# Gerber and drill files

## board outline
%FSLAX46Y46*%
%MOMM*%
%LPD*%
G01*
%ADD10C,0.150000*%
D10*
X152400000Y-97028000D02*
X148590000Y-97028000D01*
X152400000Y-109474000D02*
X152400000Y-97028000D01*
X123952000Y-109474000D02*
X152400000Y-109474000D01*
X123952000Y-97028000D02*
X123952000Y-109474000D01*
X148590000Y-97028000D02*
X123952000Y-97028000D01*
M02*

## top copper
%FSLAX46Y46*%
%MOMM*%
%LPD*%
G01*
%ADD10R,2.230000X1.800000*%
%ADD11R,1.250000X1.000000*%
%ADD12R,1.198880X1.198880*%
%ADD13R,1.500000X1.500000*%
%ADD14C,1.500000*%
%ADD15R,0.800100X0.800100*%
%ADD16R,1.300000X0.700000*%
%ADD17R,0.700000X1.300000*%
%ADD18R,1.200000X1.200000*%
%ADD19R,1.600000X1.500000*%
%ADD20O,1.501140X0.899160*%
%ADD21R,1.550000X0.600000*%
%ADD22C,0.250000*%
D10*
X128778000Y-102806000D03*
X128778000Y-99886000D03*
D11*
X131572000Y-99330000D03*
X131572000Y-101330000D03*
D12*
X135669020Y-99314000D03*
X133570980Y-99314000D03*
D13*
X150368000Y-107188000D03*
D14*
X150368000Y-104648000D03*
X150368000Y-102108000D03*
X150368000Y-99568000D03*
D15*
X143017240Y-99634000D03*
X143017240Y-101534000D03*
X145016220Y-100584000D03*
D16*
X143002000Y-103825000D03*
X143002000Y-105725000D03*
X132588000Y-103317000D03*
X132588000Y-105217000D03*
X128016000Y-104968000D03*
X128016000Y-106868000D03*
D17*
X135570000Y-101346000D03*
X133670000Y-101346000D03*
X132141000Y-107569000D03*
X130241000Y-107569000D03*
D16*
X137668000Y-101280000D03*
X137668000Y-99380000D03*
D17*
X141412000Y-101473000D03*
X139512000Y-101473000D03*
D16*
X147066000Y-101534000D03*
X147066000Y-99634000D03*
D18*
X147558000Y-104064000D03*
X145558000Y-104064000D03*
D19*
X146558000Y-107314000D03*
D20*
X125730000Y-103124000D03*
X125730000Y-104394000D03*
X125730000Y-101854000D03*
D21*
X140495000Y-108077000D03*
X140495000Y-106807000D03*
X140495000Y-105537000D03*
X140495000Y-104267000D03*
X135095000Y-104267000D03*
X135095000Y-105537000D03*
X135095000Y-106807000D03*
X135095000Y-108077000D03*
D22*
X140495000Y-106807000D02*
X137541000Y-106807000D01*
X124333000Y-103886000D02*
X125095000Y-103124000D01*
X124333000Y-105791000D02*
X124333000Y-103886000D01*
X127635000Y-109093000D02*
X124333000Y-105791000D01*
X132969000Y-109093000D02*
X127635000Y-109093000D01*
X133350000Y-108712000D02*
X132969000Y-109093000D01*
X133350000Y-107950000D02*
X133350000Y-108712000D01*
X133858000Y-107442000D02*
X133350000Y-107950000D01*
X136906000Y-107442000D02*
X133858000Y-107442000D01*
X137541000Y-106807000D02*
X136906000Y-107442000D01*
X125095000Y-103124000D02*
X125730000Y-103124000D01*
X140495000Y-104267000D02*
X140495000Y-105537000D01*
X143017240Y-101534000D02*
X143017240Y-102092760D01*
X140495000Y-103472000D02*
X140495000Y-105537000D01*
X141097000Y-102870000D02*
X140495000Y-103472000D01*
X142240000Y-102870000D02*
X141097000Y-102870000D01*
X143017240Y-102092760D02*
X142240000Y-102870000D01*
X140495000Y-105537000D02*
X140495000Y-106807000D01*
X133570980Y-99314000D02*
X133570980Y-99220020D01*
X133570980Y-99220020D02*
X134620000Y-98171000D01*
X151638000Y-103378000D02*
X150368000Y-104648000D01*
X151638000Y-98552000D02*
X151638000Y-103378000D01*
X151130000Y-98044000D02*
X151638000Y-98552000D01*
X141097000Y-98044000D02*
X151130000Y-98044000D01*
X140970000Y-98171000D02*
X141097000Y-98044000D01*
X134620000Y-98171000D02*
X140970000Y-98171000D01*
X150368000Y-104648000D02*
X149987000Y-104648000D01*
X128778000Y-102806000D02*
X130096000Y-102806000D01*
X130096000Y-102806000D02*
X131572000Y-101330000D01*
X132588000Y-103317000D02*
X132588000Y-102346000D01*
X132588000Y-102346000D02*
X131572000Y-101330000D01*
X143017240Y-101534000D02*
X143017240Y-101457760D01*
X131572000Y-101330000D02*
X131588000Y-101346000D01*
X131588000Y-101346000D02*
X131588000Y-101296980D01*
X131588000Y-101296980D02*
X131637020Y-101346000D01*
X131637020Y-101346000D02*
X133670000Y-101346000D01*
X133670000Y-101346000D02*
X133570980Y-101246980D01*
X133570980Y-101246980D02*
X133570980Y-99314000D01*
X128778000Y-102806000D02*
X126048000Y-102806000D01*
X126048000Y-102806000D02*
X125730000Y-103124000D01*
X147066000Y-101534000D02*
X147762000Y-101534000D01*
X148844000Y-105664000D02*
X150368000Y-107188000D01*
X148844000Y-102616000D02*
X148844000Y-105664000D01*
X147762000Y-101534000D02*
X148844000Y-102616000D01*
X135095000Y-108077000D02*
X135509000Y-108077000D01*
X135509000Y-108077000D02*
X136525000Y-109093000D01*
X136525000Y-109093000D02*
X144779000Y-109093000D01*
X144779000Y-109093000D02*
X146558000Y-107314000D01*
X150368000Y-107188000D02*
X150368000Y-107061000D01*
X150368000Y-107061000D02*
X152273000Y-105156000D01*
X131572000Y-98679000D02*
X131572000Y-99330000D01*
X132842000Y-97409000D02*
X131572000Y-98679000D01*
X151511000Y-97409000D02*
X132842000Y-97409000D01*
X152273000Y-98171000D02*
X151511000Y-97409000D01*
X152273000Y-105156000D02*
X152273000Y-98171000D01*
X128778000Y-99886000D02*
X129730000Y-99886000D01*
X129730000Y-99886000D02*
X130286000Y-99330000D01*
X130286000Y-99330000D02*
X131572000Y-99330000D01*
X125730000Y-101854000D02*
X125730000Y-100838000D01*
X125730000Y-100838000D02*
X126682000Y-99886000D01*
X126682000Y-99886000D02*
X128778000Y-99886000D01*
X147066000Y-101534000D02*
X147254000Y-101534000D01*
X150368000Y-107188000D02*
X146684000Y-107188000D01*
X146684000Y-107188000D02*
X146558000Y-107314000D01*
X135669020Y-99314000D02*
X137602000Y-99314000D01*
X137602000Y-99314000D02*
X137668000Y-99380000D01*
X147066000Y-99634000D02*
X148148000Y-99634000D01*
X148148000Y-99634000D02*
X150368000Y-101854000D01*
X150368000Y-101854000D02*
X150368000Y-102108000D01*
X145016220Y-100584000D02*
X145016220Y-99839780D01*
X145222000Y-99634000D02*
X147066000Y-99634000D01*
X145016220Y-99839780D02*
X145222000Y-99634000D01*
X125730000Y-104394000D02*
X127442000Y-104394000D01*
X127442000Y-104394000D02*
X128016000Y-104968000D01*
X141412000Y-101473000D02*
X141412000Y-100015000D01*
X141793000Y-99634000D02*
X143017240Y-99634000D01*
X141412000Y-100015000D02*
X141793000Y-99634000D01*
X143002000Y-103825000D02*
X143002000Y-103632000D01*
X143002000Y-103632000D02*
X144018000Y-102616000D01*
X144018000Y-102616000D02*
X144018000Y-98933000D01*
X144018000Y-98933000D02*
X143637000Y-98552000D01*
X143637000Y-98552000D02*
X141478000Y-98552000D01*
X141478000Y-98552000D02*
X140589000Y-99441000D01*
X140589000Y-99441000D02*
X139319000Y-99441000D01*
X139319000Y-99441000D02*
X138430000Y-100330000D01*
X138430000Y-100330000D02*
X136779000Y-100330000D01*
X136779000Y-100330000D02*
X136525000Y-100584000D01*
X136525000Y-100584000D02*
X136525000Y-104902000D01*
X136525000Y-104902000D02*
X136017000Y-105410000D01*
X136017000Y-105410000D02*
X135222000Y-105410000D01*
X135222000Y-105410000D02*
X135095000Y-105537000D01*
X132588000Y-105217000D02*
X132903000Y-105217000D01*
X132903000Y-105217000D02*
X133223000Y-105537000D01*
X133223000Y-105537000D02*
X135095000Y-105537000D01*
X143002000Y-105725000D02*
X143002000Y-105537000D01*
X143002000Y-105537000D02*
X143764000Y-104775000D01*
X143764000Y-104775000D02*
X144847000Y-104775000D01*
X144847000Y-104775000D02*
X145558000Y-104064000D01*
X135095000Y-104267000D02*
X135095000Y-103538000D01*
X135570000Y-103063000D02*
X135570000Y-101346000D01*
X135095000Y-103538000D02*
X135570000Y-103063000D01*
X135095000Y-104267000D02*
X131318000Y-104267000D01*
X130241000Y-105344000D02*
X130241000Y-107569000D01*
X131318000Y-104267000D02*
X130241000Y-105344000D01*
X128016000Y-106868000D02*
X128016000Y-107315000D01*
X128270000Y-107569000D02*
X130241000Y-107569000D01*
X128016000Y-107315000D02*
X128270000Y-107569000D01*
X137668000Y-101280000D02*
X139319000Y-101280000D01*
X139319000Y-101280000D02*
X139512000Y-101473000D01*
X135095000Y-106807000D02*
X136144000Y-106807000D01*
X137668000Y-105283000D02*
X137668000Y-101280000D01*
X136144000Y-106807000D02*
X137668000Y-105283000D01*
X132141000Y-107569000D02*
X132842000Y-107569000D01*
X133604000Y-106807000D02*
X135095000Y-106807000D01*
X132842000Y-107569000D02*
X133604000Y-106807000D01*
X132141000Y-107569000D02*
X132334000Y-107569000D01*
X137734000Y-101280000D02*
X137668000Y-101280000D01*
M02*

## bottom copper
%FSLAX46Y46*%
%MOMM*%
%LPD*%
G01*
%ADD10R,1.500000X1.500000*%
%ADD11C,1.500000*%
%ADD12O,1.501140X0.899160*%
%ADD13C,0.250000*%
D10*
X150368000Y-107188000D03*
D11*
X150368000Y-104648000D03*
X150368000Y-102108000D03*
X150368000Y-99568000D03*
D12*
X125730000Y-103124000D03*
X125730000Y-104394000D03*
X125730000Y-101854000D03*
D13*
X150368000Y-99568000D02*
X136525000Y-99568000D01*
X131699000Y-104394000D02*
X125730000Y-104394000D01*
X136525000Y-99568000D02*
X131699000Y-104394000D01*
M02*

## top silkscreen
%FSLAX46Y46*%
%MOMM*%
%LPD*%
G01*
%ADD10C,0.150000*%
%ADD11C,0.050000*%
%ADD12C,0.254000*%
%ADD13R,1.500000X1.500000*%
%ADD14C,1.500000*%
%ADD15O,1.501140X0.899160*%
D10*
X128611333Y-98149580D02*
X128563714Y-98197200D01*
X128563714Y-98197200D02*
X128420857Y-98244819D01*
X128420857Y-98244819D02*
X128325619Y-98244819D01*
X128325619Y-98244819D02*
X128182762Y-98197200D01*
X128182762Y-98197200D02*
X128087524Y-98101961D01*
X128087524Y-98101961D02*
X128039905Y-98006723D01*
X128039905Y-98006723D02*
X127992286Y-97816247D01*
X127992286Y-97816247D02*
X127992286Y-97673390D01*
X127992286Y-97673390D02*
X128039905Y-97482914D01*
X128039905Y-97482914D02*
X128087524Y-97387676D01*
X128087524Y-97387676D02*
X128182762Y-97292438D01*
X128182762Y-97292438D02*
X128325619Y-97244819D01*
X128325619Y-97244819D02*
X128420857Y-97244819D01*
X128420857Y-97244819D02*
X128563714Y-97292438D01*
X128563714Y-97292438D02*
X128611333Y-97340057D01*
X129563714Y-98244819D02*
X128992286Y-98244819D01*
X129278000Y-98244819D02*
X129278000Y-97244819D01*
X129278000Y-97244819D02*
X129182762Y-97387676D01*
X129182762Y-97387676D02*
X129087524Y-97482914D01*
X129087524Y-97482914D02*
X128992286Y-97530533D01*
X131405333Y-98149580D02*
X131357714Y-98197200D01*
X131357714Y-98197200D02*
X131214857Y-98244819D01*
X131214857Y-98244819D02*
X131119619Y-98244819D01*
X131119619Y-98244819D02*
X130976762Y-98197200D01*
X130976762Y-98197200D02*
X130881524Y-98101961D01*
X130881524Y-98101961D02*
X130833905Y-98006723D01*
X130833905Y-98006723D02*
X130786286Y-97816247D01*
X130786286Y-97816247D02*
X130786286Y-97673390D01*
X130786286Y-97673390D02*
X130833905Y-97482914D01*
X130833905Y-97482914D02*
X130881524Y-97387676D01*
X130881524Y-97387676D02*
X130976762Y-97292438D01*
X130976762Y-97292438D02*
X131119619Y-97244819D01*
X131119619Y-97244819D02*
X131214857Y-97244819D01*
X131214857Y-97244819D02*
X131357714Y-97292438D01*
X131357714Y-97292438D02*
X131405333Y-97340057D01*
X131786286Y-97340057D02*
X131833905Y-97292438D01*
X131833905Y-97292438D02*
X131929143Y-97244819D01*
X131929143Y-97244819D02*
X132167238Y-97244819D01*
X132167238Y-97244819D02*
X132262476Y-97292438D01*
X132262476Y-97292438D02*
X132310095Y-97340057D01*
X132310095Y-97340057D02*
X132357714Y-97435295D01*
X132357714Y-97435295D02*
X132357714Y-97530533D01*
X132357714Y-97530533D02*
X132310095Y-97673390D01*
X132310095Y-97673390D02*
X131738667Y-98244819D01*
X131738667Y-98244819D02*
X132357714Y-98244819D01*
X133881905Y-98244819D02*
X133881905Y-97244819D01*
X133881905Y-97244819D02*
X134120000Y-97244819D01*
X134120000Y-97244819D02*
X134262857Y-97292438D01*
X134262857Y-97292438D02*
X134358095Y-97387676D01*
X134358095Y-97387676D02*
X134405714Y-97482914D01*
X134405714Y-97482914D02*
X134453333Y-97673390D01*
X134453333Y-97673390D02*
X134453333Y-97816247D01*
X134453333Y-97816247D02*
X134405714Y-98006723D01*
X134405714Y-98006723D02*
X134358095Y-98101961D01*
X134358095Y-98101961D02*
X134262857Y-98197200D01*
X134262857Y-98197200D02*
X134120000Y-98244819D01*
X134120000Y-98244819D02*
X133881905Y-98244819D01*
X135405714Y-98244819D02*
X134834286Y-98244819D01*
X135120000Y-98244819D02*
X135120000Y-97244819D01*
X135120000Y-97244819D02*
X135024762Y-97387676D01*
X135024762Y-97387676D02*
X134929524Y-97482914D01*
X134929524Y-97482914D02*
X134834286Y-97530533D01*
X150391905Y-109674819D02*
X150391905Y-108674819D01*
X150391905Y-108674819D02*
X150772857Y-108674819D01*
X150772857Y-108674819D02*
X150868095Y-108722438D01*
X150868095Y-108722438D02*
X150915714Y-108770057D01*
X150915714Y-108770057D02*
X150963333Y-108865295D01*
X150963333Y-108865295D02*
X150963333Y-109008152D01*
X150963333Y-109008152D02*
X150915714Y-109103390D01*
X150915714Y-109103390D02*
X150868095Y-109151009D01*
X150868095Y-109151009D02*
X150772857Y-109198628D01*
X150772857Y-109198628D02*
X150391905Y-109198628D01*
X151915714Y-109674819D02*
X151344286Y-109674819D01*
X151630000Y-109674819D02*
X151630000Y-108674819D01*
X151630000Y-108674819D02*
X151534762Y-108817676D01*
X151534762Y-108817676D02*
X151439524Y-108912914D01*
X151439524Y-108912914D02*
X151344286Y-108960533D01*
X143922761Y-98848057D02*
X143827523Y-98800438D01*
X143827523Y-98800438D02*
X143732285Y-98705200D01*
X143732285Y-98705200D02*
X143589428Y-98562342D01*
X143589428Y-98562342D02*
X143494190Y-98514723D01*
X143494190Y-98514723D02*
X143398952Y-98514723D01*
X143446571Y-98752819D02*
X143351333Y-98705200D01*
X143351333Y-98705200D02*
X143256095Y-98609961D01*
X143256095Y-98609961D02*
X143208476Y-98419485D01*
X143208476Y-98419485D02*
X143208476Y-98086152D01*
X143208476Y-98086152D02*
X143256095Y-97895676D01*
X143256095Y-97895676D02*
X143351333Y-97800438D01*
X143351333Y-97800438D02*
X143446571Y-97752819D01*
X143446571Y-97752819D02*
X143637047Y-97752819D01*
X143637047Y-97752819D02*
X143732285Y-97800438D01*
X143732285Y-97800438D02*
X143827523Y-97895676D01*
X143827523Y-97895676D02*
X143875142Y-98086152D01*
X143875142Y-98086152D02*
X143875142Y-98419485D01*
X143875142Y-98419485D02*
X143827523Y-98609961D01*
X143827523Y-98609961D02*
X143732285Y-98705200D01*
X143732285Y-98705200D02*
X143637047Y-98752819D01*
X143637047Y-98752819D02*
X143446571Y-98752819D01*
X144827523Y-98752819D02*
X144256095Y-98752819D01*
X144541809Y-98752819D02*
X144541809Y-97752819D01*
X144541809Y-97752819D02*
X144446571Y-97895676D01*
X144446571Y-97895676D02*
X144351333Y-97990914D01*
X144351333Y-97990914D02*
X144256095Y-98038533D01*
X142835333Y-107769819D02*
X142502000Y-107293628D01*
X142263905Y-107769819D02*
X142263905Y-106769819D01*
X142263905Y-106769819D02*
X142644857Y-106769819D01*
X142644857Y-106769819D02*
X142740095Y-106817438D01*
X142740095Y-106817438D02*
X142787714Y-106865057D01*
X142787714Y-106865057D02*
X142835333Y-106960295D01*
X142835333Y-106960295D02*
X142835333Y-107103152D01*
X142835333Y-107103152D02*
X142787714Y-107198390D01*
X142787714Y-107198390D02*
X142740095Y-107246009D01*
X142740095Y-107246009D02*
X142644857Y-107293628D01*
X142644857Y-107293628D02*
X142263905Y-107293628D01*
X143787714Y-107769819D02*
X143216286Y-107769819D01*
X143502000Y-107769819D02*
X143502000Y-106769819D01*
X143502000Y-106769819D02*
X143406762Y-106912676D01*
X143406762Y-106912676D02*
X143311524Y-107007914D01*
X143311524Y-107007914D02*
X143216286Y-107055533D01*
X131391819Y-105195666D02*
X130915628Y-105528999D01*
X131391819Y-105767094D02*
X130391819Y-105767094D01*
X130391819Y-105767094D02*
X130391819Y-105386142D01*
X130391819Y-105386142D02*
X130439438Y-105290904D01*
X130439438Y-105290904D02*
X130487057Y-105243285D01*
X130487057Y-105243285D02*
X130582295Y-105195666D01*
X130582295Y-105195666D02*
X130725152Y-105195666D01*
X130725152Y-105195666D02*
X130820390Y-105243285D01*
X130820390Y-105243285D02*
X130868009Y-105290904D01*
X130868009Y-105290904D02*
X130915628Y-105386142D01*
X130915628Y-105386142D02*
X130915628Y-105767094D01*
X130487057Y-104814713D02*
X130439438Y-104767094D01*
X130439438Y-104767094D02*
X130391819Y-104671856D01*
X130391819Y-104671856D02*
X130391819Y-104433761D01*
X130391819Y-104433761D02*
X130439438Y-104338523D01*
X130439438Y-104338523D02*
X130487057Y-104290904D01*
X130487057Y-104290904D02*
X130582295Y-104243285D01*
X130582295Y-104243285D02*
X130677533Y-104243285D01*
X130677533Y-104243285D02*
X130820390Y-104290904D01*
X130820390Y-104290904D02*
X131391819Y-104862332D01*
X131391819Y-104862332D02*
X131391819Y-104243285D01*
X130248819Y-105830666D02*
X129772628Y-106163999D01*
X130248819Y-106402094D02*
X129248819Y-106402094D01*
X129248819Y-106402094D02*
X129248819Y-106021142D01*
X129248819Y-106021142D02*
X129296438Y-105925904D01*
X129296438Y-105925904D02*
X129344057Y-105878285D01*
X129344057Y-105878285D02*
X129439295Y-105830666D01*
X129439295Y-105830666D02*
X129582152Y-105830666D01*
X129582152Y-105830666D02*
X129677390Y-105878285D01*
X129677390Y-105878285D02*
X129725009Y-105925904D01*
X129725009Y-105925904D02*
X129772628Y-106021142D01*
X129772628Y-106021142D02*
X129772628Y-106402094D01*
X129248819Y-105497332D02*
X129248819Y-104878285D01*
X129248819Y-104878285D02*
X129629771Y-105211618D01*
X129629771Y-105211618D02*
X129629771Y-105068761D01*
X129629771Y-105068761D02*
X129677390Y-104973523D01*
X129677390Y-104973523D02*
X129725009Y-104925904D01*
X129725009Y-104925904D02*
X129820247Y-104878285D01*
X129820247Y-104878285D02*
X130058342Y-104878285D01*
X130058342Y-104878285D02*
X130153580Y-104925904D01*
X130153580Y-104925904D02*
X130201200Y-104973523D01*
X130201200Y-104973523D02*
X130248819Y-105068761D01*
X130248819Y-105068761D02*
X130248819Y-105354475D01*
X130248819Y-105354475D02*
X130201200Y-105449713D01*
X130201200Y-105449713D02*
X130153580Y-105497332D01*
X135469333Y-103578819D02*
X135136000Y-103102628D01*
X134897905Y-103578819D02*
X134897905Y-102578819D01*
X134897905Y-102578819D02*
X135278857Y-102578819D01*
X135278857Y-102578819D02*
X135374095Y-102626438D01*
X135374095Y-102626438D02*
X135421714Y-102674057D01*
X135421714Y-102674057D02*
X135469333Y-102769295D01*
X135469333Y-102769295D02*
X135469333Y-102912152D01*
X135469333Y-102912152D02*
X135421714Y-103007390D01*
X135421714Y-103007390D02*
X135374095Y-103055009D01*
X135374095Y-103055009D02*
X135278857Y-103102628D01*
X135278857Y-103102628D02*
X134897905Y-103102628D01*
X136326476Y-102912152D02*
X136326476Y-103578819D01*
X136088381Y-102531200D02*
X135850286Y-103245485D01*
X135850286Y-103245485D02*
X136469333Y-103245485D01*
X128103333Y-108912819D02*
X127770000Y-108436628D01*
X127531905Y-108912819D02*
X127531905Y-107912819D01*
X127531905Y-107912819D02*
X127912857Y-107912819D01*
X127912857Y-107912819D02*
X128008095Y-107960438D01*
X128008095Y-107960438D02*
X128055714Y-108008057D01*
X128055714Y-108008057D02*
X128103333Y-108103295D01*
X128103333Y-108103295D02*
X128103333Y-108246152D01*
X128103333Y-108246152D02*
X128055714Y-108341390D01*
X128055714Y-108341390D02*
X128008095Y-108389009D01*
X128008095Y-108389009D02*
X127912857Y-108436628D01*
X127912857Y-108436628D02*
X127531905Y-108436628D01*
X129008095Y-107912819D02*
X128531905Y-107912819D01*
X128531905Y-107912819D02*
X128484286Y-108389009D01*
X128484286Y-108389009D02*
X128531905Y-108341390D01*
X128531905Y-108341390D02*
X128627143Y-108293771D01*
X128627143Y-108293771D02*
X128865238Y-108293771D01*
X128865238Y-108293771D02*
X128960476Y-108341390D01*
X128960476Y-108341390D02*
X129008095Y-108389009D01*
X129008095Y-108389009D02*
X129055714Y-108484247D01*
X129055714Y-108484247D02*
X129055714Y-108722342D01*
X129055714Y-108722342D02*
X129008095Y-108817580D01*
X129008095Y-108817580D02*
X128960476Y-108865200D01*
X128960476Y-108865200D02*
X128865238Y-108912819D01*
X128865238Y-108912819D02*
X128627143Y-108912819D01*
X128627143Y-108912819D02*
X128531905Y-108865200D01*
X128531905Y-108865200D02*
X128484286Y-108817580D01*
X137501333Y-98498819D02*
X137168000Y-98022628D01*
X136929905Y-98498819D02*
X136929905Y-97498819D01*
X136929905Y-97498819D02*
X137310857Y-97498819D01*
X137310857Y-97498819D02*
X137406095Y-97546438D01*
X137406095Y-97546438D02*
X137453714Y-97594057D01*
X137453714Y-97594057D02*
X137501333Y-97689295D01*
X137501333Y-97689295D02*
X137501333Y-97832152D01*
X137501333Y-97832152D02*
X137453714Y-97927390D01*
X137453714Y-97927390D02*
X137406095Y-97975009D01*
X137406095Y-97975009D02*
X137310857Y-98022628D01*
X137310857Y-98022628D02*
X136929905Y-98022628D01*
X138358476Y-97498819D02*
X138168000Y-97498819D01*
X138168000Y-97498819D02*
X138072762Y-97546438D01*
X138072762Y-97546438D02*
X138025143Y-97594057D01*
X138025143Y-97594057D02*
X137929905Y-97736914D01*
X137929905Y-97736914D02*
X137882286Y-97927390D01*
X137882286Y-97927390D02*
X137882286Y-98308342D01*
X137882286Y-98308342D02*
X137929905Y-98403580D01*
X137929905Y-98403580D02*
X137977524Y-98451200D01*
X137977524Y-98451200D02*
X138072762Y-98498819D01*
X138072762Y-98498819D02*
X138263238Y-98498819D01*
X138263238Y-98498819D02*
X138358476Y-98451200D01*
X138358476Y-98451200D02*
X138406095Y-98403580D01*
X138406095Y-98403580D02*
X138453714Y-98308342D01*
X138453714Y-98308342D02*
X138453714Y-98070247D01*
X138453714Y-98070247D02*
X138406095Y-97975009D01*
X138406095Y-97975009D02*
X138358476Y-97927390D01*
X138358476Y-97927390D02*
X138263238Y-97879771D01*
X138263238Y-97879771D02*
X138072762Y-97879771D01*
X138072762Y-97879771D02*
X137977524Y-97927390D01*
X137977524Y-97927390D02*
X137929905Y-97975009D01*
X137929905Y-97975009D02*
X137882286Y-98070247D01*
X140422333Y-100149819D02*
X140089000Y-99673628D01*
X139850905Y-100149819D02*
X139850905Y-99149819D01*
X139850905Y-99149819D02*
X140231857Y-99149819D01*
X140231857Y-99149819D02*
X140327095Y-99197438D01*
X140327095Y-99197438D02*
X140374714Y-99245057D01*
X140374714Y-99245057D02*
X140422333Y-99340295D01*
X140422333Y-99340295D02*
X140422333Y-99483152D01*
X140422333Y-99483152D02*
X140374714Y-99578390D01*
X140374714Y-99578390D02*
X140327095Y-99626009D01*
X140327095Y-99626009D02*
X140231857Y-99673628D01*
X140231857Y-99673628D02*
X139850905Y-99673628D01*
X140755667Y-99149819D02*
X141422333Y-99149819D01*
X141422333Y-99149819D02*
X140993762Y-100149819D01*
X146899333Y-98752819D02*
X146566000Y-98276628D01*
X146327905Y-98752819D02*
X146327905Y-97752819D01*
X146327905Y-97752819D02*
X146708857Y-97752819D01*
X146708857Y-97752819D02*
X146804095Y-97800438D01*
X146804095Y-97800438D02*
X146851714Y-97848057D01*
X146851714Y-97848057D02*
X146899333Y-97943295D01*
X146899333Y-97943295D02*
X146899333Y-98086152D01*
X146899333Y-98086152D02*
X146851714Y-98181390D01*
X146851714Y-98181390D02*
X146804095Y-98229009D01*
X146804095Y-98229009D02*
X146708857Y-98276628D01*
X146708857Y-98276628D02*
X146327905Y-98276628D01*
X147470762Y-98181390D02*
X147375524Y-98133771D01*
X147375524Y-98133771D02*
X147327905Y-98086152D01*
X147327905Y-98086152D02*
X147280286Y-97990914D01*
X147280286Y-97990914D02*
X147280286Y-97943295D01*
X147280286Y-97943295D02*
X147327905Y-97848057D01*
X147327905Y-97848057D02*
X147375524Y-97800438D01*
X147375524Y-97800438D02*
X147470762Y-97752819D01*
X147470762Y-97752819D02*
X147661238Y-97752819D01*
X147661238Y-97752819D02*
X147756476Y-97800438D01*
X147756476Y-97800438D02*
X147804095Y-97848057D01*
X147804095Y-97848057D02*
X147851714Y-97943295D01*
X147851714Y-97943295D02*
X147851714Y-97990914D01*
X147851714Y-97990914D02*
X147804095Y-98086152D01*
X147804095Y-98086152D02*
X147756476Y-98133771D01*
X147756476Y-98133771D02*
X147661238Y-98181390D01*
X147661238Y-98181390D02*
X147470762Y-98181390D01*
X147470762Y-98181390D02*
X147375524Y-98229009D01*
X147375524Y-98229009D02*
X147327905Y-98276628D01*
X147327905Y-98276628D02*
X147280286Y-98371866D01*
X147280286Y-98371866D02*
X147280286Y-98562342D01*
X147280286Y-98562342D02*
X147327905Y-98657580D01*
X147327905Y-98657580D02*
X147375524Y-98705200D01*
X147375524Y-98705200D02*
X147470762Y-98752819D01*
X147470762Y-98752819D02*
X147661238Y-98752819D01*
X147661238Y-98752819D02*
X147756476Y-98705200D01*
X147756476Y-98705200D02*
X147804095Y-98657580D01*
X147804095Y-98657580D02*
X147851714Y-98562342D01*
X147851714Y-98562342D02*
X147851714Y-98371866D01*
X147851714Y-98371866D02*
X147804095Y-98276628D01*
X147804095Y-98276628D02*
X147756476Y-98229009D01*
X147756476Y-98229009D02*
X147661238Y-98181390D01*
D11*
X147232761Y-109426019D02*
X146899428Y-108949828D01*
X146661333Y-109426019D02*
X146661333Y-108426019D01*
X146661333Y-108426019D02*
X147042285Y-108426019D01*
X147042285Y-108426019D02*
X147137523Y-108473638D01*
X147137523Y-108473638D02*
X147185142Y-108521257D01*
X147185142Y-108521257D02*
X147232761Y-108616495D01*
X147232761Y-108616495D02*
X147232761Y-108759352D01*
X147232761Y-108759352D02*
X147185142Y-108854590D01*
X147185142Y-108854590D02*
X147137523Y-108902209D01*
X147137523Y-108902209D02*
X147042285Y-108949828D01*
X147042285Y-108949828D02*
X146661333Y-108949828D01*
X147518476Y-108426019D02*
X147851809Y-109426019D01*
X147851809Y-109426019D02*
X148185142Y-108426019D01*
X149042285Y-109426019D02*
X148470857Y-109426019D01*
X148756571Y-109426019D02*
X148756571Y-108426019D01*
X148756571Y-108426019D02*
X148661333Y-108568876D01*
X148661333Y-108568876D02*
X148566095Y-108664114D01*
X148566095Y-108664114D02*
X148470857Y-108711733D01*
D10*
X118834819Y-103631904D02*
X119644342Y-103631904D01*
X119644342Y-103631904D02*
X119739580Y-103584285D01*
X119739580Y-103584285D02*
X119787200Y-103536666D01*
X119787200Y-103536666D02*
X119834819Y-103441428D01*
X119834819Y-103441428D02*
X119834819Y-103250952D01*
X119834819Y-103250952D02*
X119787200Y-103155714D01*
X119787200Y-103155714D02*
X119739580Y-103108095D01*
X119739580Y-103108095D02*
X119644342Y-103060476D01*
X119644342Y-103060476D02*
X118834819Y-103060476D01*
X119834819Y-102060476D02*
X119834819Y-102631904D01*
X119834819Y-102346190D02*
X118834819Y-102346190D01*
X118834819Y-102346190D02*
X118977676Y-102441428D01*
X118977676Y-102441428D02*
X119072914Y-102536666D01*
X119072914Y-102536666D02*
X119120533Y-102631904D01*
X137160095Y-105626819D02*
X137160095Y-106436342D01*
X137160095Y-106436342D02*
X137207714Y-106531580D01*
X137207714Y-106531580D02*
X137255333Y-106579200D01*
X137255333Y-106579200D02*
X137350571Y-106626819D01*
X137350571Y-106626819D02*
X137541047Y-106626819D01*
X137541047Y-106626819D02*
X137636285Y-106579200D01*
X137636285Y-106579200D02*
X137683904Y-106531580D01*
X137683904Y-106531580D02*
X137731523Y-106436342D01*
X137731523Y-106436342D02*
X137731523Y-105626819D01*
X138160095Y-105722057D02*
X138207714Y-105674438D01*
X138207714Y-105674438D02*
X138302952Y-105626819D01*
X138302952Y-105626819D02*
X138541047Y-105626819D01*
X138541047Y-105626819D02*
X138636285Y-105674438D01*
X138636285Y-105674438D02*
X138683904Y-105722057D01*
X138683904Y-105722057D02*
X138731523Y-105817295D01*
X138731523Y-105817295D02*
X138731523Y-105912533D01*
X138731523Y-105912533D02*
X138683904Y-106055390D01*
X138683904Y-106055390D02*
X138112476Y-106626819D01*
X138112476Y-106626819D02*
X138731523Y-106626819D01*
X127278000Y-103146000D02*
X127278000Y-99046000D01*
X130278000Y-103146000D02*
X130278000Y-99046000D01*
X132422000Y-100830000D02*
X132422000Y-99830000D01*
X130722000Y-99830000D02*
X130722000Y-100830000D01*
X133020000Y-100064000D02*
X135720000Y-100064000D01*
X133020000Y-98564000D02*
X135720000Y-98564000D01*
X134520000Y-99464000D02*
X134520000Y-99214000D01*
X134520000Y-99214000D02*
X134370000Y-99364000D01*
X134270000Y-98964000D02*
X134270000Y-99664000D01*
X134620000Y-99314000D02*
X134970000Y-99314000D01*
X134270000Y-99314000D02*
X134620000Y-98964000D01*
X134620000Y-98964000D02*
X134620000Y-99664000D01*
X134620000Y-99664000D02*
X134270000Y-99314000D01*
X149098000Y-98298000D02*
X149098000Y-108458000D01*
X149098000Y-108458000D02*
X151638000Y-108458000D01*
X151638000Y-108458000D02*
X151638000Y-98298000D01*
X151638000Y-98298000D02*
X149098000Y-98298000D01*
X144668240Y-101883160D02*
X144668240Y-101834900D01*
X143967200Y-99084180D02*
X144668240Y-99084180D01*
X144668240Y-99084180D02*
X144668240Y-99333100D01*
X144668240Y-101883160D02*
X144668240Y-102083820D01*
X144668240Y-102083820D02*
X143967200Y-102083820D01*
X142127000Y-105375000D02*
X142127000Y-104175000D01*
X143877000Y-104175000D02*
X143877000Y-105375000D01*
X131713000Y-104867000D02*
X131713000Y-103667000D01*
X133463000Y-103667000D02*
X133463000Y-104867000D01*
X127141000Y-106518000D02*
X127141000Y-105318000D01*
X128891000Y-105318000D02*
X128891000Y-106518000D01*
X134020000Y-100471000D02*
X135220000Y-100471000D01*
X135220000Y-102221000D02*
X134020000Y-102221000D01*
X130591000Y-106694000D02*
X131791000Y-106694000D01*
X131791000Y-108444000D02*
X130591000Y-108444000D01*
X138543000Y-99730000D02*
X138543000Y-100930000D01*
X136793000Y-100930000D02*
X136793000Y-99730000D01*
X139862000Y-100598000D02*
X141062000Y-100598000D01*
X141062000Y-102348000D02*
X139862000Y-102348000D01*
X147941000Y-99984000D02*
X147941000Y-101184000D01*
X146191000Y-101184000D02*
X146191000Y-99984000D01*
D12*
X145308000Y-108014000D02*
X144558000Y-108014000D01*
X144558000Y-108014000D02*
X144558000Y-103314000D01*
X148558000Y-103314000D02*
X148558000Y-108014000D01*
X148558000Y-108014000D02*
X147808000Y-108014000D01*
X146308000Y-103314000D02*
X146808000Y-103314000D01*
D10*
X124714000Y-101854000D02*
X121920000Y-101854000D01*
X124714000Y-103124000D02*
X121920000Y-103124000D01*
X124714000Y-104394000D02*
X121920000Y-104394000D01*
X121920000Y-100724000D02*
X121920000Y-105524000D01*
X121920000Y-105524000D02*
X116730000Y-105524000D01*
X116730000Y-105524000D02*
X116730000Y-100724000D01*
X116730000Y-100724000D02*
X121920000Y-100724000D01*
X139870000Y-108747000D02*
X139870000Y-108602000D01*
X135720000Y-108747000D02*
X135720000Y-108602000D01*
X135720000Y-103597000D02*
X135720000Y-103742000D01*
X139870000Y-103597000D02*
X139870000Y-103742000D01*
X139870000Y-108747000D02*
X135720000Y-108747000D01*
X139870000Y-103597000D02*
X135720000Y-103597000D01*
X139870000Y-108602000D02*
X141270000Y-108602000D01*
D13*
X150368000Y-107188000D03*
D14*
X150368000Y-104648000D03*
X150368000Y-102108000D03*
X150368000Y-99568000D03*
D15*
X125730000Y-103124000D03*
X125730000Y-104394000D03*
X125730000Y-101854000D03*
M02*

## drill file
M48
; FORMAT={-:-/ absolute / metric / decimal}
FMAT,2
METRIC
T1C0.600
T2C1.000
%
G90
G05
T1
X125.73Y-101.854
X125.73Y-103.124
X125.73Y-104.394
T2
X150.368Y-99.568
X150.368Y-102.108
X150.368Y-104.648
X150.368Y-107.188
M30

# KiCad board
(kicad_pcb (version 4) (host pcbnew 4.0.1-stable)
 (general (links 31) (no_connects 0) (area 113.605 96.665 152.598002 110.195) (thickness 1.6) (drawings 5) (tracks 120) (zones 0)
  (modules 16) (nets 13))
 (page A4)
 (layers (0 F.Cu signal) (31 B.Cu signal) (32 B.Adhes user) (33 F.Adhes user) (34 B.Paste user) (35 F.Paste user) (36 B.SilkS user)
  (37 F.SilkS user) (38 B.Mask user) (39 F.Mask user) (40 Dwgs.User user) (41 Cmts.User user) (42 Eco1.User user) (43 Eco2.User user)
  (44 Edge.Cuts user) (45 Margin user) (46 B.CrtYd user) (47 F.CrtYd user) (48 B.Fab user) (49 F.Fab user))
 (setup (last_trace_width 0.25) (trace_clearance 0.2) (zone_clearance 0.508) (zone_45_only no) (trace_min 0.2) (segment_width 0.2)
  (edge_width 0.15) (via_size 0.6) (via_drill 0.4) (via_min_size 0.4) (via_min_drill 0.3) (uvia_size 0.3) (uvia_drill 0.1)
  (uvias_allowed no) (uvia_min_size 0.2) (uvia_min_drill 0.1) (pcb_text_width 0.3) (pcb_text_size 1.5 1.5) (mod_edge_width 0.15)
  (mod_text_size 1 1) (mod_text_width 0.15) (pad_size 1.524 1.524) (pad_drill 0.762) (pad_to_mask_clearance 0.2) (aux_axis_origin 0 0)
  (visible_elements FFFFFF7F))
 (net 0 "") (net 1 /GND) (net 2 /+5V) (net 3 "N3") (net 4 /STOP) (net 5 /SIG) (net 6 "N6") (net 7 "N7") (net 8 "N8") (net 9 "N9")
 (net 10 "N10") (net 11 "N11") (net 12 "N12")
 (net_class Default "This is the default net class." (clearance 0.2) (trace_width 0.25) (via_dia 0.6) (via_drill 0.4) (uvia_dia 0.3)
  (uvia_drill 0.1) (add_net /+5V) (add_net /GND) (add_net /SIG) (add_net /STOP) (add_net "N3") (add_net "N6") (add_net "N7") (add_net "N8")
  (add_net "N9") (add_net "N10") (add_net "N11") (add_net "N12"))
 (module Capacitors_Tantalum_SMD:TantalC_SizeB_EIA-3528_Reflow (layer F.Cu) (at 128.778 101.346 270)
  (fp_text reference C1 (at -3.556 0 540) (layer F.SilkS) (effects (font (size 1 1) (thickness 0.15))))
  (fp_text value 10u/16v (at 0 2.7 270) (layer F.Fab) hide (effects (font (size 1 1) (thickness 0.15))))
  (fp_line (start 1.8 1.5) (end -2.3 1.5) (layer F.SilkS) (width 0.15))
  (fp_line (start 1.8 -1.5) (end -2.3 -1.5) (layer F.SilkS) (width 0.15))
  (pad 2 smd rect (at 1.46 0 270) (size 1.8 2.23) (layers F.Cu F.Paste F.Mask) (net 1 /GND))
  (pad 1 smd rect (at -1.46 0 270) (size 1.8 2.23) (layers F.Cu F.Paste F.Mask) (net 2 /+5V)))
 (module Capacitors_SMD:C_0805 (layer F.Cu) (at 131.572 100.33 270)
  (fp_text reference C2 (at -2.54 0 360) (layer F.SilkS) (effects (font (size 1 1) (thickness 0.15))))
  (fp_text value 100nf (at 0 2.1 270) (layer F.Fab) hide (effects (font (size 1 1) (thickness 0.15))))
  (fp_line (start 0.5 -0.85) (end -0.5 -0.85) (layer F.SilkS) (width 0.15))
  (fp_line (start -0.5 0.85) (end 0.5 0.85) (layer F.SilkS) (width 0.15))
  (pad 1 smd rect (at -1 0 270) (size 1 1.25) (layers F.Cu F.Paste F.Mask) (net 2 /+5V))
  (pad 2 smd rect (at 1 0 270) (size 1 1.25) (layers F.Cu F.Paste F.Mask) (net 1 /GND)))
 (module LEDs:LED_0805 (layer F.Cu) (at 134.62 99.314)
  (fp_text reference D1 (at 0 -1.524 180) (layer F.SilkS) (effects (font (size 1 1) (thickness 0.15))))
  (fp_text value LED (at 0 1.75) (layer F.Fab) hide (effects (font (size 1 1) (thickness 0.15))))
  (fp_line (start -1.6 0.75) (end 1.1 0.75) (layer F.SilkS) (width 0.15))
  (fp_line (start -1.6 -0.75) (end 1.1 -0.75) (layer F.SilkS) (width 0.15))
  (fp_line (start -0.1 0.15) (end -0.1 -0.1) (layer F.SilkS) (width 0.15))
  (fp_line (start -0.1 -0.1) (end -0.25 0.05) (layer F.SilkS) (width 0.15))
  (fp_line (start -0.35 -0.35) (end -0.35 0.35) (layer F.SilkS) (width 0.15))
  (fp_line (start 0 0) (end 0.35 0) (layer F.SilkS) (width 0.15))
  (fp_line (start -0.35 0) (end 0 -0.35) (layer F.SilkS) (width 0.15))
  (fp_line (start 0 -0.35) (end 0 0.35) (layer F.SilkS) (width 0.15))
  (fp_line (start 0 0.35) (end -0.35 0) (layer F.SilkS) (width 0.15))
  (pad 2 smd rect (at 1.04902 0 180) (size 1.19888 1.19888) (layers F.Cu F.Paste F.Mask) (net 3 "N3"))
  (pad 1 smd rect (at -1.04902 0 180) (size 1.19888 1.19888) (layers F.Cu F.Paste F.Mask) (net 1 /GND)))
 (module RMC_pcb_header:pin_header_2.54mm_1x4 (layer F.Cu) (at 150.368 103.378 90)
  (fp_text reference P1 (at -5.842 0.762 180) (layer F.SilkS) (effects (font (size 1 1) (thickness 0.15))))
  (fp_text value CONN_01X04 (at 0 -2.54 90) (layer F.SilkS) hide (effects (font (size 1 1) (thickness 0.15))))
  (fp_line (start 5.08 -1.27) (end -5.08 -1.27) (layer F.SilkS) (width 0.15))
  (fp_line (start -5.08 -1.27) (end -5.08 1.27) (layer F.SilkS) (width 0.15))
  (fp_line (start -5.08 1.27) (end 5.08 1.27) (layer F.SilkS) (width 0.15))
  (fp_line (start 5.08 1.27) (end 5.08 -1.27) (layer F.SilkS) (width 0.15))
  (pad 1 thru_hole rect (at -3.81 0 90) (size 1.5 1.5) (drill 1) (layers *.Cu *.Mask F.SilkS) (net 2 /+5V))
  (pad 2 thru_hole circle (at -1.27 0 90) (size 1.5 1.5) (drill 1) (layers *.Cu *.Mask F.SilkS) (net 1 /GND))
  (pad 3 thru_hole circle (at 1.27 0 90) (size 1.5 1.5) (drill 1) (layers *.Cu *.Mask F.SilkS) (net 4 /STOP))
  (pad 4 thru_hole circle (at 3.81 0 90) (size 1.5 1.5) (drill 1) (layers *.Cu *.Mask F.SilkS) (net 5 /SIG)))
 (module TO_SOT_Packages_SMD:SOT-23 (layer F.Cu) (at 144.018 100.584 270)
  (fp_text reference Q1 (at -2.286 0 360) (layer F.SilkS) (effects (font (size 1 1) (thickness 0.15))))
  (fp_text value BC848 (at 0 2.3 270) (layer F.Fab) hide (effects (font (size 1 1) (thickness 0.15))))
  (fp_line (start 1.29916 -0.65024) (end 1.2509 -0.65024) (layer F.SilkS) (width 0.15))
  (fp_line (start -1.49982 0.0508) (end -1.49982 -0.65024) (layer F.SilkS) (width 0.15))
  (fp_line (start -1.49982 -0.65024) (end -1.2509 -0.65024) (layer F.SilkS) (width 0.15))
  (fp_line (start 1.29916 -0.65024) (end 1.49982 -0.65024) (layer F.SilkS) (width 0.15))
  (fp_line (start 1.49982 -0.65024) (end 1.49982 0.0508) (layer F.SilkS) (width 0.15))
  (pad 1 smd rect (at -0.95 1.00076 270) (size 0.8001 0.8001) (layers F.Cu F.Paste F.Mask) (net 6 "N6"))
  (pad 2 smd rect (at 0.95 1.00076 270) (size 0.8001 0.8001) (layers F.Cu F.Paste F.Mask) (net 1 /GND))
  (pad 3 smd rect (at 0 -0.99822 270) (size 0.8001 0.8001) (layers F.Cu F.Paste F.Mask) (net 4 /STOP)))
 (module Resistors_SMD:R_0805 (layer F.Cu) (at 143.002 104.775 270)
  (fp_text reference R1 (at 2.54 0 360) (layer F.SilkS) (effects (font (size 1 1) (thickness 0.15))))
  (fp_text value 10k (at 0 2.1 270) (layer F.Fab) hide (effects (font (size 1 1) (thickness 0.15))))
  (fp_line (start 0.6 0.875) (end -0.6 0.875) (layer F.SilkS) (width 0.15))
  (fp_line (start -0.6 -0.875) (end 0.6 -0.875) (layer F.SilkS) (width 0.15))
  (pad 1 smd rect (at -0.95 0 270) (size 0.7 1.3) (layers F.Cu F.Paste F.Mask) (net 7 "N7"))
  (pad 2 smd rect (at 0.95 0 270) (size 0.7 1.3) (layers F.Cu F.Paste F.Mask) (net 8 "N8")))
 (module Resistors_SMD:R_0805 (layer F.Cu) (at 132.588 104.267 270)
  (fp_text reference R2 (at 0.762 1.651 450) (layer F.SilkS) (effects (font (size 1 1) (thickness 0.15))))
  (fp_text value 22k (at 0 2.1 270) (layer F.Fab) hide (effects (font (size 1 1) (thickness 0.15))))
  (fp_line (start 0.6 0.875) (end -0.6 0.875) (layer F.SilkS) (width 0.15))
  (fp_line (start -0.6 -0.875) (end 0.6 -0.875) (layer F.SilkS) (width 0.15))
  (pad 1 smd rect (at -0.95 0 270) (size 0.7 1.3) (layers F.Cu F.Paste F.Mask) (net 1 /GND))
  (pad 2 smd rect (at 0.95 0 270) (size 0.7 1.3) (layers F.Cu F.Paste F.Mask) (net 7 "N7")))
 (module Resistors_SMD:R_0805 (layer F.Cu) (at 128.016 105.918 270)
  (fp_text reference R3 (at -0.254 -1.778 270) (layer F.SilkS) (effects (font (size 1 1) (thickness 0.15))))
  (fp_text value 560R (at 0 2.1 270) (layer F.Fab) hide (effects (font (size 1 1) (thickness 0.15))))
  (fp_line (start 0.6 0.875) (end -0.6 0.875) (layer F.SilkS) (width 0.15))
  (fp_line (start -0.6 -0.875) (end 0.6 -0.875) (layer F.SilkS) (width 0.15))
  (pad 1 smd rect (at -0.95 0 270) (size 0.7 1.3) (layers F.Cu F.Paste F.Mask) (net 5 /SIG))
  (pad 2 smd rect (at 0.95 0 270) (size 0.7 1.3) (layers F.Cu F.Paste F.Mask) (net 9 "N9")))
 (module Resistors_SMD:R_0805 (layer F.Cu) (at 134.62 101.346 180)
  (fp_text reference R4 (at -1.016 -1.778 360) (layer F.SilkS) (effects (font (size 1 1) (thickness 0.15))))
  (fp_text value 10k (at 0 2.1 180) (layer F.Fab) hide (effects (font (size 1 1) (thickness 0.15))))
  (fp_line (start 0.6 0.875) (end -0.6 0.875) (layer F.SilkS) (width 0.15))
  (fp_line (start -0.6 -0.875) (end 0.6 -0.875) (layer F.SilkS) (width 0.15))
  (pad 1 smd rect (at -0.95 0 180) (size 0.7 1.3) (layers F.Cu F.Paste F.Mask) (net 9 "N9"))
  (pad 2 smd rect (at 0.95 0 180) (size 0.7 1.3) (layers F.Cu F.Paste F.Mask) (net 1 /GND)))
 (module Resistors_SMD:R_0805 (layer F.Cu) (at 131.191 107.569 180)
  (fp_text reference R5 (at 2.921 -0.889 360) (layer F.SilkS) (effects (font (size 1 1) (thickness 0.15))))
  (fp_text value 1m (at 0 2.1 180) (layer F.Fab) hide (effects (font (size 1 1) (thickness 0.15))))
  (fp_line (start 0.6 0.875) (end -0.6 0.875) (layer F.SilkS) (width 0.15))
  (fp_line (start -0.6 -0.875) (end 0.6 -0.875) (layer F.SilkS) (width 0.15))
  (pad 1 smd rect (at -0.95 0 180) (size 0.7 1.3) (layers F.Cu F.Paste F.Mask) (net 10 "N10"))
  (pad 2 smd rect (at 0.95 0 180) (size 0.7 1.3) (layers F.Cu F.Paste F.Mask) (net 9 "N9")))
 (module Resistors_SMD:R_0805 (layer F.Cu) (at 137.668 100.33 90)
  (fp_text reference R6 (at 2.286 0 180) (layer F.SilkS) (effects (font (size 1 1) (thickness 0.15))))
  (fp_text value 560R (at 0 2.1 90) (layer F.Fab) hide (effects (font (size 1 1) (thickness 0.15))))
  (fp_line (start 0.6 0.875) (end -0.6 0.875) (layer F.SilkS) (width 0.15))
  (fp_line (start -0.6 -0.875) (end 0.6 -0.875) (layer F.SilkS) (width 0.15))
  (pad 1 smd rect (at -0.95 0 90) (size 0.7 1.3) (layers F.Cu F.Paste F.Mask) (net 10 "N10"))
  (pad 2 smd rect (at 0.95 0 90) (size 0.7 1.3) (layers F.Cu F.Paste F.Mask) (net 3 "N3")))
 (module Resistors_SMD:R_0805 (layer F.Cu) (at 140.462 101.473 180)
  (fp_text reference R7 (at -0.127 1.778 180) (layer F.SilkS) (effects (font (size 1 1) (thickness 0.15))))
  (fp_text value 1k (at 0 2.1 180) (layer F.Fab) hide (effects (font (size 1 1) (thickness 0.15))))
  (fp_line (start 0.6 0.875) (end -0.6 0.875) (layer F.SilkS) (width 0.15))
  (fp_line (start -0.6 -0.875) (end 0.6 -0.875) (layer F.SilkS) (width 0.15))
  (pad 1 smd rect (at -0.95 0 180) (size 0.7 1.3) (layers F.Cu F.Paste F.Mask) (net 6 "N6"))
  (pad 2 smd rect (at 0.95 0 180) (size 0.7 1.3) (layers F.Cu F.Paste F.Mask) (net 10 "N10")))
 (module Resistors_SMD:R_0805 (layer F.Cu) (at 147.066 100.584 90)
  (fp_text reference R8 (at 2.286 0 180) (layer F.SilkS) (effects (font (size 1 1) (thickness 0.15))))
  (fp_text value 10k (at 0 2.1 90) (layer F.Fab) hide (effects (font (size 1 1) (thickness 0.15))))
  (fp_line (start 0.6 0.875) (end -0.6 0.875) (layer F.SilkS) (width 0.15))
  (fp_line (start -0.6 -0.875) (end 0.6 -0.875) (layer F.SilkS) (width 0.15))
  (pad 1 smd rect (at -0.95 0 90) (size 0.7 1.3) (layers F.Cu F.Paste F.Mask) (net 2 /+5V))
  (pad 2 smd rect (at 0.95 0 90) (size 0.7 1.3) (layers F.Cu F.Paste F.Mask) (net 4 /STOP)))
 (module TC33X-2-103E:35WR (layer F.Cu) (at 146.558 105.664 180) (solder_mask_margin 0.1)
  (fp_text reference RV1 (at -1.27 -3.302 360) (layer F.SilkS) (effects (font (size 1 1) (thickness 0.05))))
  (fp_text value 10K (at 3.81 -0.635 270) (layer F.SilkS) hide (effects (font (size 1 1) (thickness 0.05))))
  (fp_line (start 1.25 -2.35) (end 2 -2.35) (layer F.SilkS) (width 0.254))
  (fp_line (start 2 -2.35) (end 2 2.35) (layer F.SilkS) (width 0.254))
  (fp_line (start -2 2.35) (end -2 -2.35) (layer F.SilkS) (width 0.254))
  (fp_line (start -2 -2.35) (end -1.25 -2.35) (layer F.SilkS) (width 0.254))
  (fp_line (start 0.25 2.35) (end -0.25 2.35) (layer F.SilkS) (width 0.254))
  (pad 1 smd rect (at -1 1.6 180) (size 1.2 1.2) (layers F.Cu F.Paste F.Mask) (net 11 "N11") (solder_mask_margin 0.2))
  (pad 3 smd rect (at 1 1.6 180) (size 1.2 1.2) (layers F.Cu F.Paste F.Mask) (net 8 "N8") (solder_mask_margin 0.2))
  (pad 2 smd rect (at 0 -1.65 180) (size 1.6 1.5) (layers F.Cu F.Paste F.Mask) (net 2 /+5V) (solder_mask_margin 0.2)))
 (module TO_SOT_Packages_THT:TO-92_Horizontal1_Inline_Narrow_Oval (layer F.Cu) (at 125.73 101.854 270)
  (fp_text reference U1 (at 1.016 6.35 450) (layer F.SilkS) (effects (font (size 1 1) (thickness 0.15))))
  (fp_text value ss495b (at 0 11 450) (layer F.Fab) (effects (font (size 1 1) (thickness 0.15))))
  (fp_line (start 0 1.016) (end 0 3.81) (layer F.SilkS) (width 0.15))
  (fp_line (start 1.27 1.016) (end 1.27 3.81) (layer F.SilkS) (width 0.15))
  (fp_line (start 2.54 1.016) (end 2.54 3.81) (layer F.SilkS) (width 0.15))
  (fp_line (start -1.13 3.81) (end 3.67 3.81) (layer F.SilkS) (width 0.15))
  (fp_line (start 3.67 3.81) (end 3.67 9) (layer F.SilkS) (width 0.15))
  (fp_line (start 3.67 9) (end -1.13 9) (layer F.SilkS) (width 0.15))
  (fp_line (start -1.13 9) (end -1.13 3.81) (layer F.SilkS) (width 0.15))
  (pad 2 thru_hole oval (at 1.27 0 90) (size 0.89916 1.50114) (drill 0.6) (layers *.Cu *.Mask F.SilkS) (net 1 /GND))
  (pad 3 thru_hole oval (at 2.54 0 90) (size 0.89916 1.50114) (drill 0.6) (layers *.Cu *.Mask F.SilkS) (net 5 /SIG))
  (pad 1 thru_hole oval (at 0 0 90) (size 0.89916 1.50114) (drill 0.6) (layers *.Cu *.Mask F.SilkS) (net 2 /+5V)))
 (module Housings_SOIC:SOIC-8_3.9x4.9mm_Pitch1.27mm (layer F.Cu) (at 137.795 106.172 180)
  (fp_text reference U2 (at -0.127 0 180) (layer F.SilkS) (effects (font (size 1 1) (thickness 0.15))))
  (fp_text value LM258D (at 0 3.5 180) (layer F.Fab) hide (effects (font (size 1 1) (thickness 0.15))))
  (fp_line (start -2.075 -2.575) (end -2.075 -2.43) (layer F.SilkS) (width 0.15))
  (fp_line (start 2.075 -2.575) (end 2.075 -2.43) (layer F.SilkS) (width 0.15))
  (fp_line (start 2.075 2.575) (end 2.075 2.43) (layer F.SilkS) (width 0.15))
  (fp_line (start -2.075 2.575) (end -2.075 2.43) (layer F.SilkS) (width 0.15))
  (fp_line (start -2.075 -2.575) (end 2.075 -2.575) (layer F.SilkS) (width 0.15))
  (fp_line (start -2.075 2.575) (end 2.075 2.575) (layer F.SilkS) (width 0.15))
  (fp_line (start -2.075 -2.43) (end -3.475 -2.43) (layer F.SilkS) (width 0.15))
  (pad 1 smd rect (at -2.7 -1.905 180) (size 1.55 0.6) (layers F.Cu F.Paste F.Mask) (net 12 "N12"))
  (pad 2 smd rect (at -2.7 -0.635 180) (size 1.55 0.6) (layers F.Cu F.Paste F.Mask) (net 1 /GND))
  (pad 3 smd rect (at -2.7 0.635 180) (size 1.55 0.6) (layers F.Cu F.Paste F.Mask) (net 1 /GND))
  (pad 4 smd rect (at -2.7 1.905 180) (size 1.55 0.6) (layers F.Cu F.Paste F.Mask) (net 1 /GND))
  (pad 5 smd rect (at 2.7 1.905 180) (size 1.55 0.6) (layers F.Cu F.Paste F.Mask) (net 9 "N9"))
  (pad 6 smd rect (at 2.7 0.635 180) (size 1.55 0.6) (layers F.Cu F.Paste F.Mask) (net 7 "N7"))
  (pad 7 smd rect (at 2.7 -0.635 180) (size 1.55 0.6) (layers F.Cu F.Paste F.Mask) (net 10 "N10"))
  (pad 8 smd rect (at 2.7 -1.905 180) (size 1.55 0.6) (layers F.Cu F.Paste F.Mask) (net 2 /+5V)))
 (gr_line (start 152.4 97.028) (end 148.59 97.028) (angle 90) (layer Edge.Cuts) (width 0.15))
 (gr_line (start 152.4 109.474) (end 152.4 97.028) (angle 90) (layer Edge.Cuts) (width 0.15))
 (gr_line (start 123.952 109.474) (end 152.4 109.474) (angle 90) (layer Edge.Cuts) (width 0.15))
 (gr_line (start 123.952 97.028) (end 123.952 109.474) (angle 90) (layer Edge.Cuts) (width 0.15))
 (gr_line (start 148.59 97.028) (end 123.952 97.028) (angle 90) (layer Edge.Cuts) (width 0.15))
 (segment (start 140.495 106.807) (end 137.541 106.807) (width 0.25) (layer F.Cu) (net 1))
 (segment (start 124.333 103.886) (end 125.095 103.124) (width 0.25) (layer F.Cu) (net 1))
 (segment (start 124.333 105.791) (end 124.333 103.886) (width 0.25) (layer F.Cu) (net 1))
 (segment (start 127.635 109.093) (end 124.333 105.791) (width 0.25) (layer F.Cu) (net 1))
 (segment (start 132.969 109.093) (end 127.635 109.093) (width 0.25) (layer F.Cu) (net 1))
 (segment (start 133.35 108.712) (end 132.969 109.093) (width 0.25) (layer F.Cu) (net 1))
 (segment (start 133.35 107.95) (end 133.35 108.712) (width 0.25) (layer F.Cu) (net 1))
 (segment (start 133.858 107.442) (end 133.35 107.95) (width 0.25) (layer F.Cu) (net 1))
 (segment (start 136.906 107.442) (end 133.858 107.442) (width 0.25) (layer F.Cu) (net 1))
 (segment (start 137.541 106.807) (end 136.906 107.442) (width 0.25) (layer F.Cu) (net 1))
 (segment (start 125.095 103.124) (end 125.73 103.124) (width 0.25) (layer F.Cu) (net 1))
 (segment (start 140.495 104.267) (end 140.495 105.537) (width 0.25) (layer F.Cu) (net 1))
 (segment (start 143.01724 101.534) (end 143.01724 102.09276) (width 0.25) (layer F.Cu) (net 1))
 (segment (start 140.495 103.472) (end 140.495 105.537) (width 0.25) (layer F.Cu) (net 1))
 (segment (start 141.097 102.87) (end 140.495 103.472) (width 0.25) (layer F.Cu) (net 1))
 (segment (start 142.24 102.87) (end 141.097 102.87) (width 0.25) (layer F.Cu) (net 1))
 (segment (start 143.01724 102.09276) (end 142.24 102.87) (width 0.25) (layer F.Cu) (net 1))
 (segment (start 140.495 105.537) (end 140.495 106.807) (width 0.25) (layer F.Cu) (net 1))
 (segment (start 133.57098 99.314) (end 133.57098 99.22002) (width 0.25) (layer F.Cu) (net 1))
 (segment (start 133.57098 99.22002) (end 134.62 98.171) (width 0.25) (layer F.Cu) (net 1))
 (segment (start 151.638 103.378) (end 150.368 104.648) (width 0.25) (layer F.Cu) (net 1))
 (segment (start 151.638 98.552) (end 151.638 103.378) (width 0.25) (layer F.Cu) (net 1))
 (segment (start 151.13 98.044) (end 151.638 98.552) (width 0.25) (layer F.Cu) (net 1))
 (segment (start 141.097 98.044) (end 151.13 98.044) (width 0.25) (layer F.Cu) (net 1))
 (segment (start 140.97 98.171) (end 141.097 98.044) (width 0.25) (layer F.Cu) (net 1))
 (segment (start 134.62 98.171) (end 140.97 98.171) (width 0.25) (layer F.Cu) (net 1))
 (segment (start 150.368 104.648) (end 149.987 104.648) (width 0.25) (layer F.Cu) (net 1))
 (segment (start 128.778 102.806) (end 130.096 102.806) (width 0.25) (layer F.Cu) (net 1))
 (segment (start 130.096 102.806) (end 131.572 101.33) (width 0.25) (layer F.Cu) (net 1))
 (segment (start 132.588 103.317) (end 132.588 102.346) (width 0.25) (layer F.Cu) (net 1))
 (segment (start 132.588 102.346) (end 131.572 101.33) (width 0.25) (layer F.Cu) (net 1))
 (segment (start 143.01724 101.534) (end 143.01724 101.45776) (width 0.25) (layer F.Cu) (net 1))
 (segment (start 131.572 101.33) (end 131.588 101.346) (width 0.25) (layer F.Cu) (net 1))
 (segment (start 131.588 101.346) (end 131.588 101.29698) (width 0.25) (layer F.Cu) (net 1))
 (segment (start 131.588 101.29698) (end 131.63702 101.346) (width 0.25) (layer F.Cu) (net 1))
 (segment (start 131.63702 101.346) (end 133.67 101.346) (width 0.25) (layer F.Cu) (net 1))
 (segment (start 133.67 101.346) (end 133.57098 101.24698) (width 0.25) (layer F.Cu) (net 1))
 (segment (start 133.57098 101.24698) (end 133.57098 99.314) (width 0.25) (layer F.Cu) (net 1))
 (segment (start 128.778 102.806) (end 126.048 102.806) (width 0.25) (layer F.Cu) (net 1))
 (segment (start 126.048 102.806) (end 125.73 103.124) (width 0.25) (layer F.Cu) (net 1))
 (segment (start 147.066 101.534) (end 147.762 101.534) (width 0.25) (layer F.Cu) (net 2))
 (segment (start 148.844 105.664) (end 150.368 107.188) (width 0.25) (layer F.Cu) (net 2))
 (segment (start 148.844 102.616) (end 148.844 105.664) (width 0.25) (layer F.Cu) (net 2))
 (segment (start 147.762 101.534) (end 148.844 102.616) (width 0.25) (layer F.Cu) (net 2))
 (segment (start 135.095 108.077) (end 135.509 108.077) (width 0.25) (layer F.Cu) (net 2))
 (segment (start 135.509 108.077) (end 136.525 109.093) (width 0.25) (layer F.Cu) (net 2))
 (segment (start 136.525 109.093) (end 144.779 109.093) (width 0.25) (layer F.Cu) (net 2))
 (segment (start 144.779 109.093) (end 146.558 107.314) (width 0.25) (layer F.Cu) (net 2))
 (segment (start 150.368 107.188) (end 150.368 107.061) (width 0.25) (layer F.Cu) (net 2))
 (segment (start 150.368 107.061) (end 152.273 105.156) (width 0.25) (layer F.Cu) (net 2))
 (segment (start 131.572 98.679) (end 131.572 99.33) (width 0.25) (layer F.Cu) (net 2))
 (segment (start 132.842 97.409) (end 131.572 98.679) (width 0.25) (layer F.Cu) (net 2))
 (segment (start 151.511 97.409) (end 132.842 97.409) (width 0.25) (layer F.Cu) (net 2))
 (segment (start 152.273 98.171) (end 151.511 97.409) (width 0.25) (layer F.Cu) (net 2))
 (segment (start 152.273 105.156) (end 152.273 98.171) (width 0.25) (layer F.Cu) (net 2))
 (segment (start 128.778 99.886) (end 129.73 99.886) (width 0.25) (layer F.Cu) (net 2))
 (segment (start 129.73 99.886) (end 130.286 99.33) (width 0.25) (layer F.Cu) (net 2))
 (segment (start 130.286 99.33) (end 131.572 99.33) (width 0.25) (layer F.Cu) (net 2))
 (segment (start 125.73 101.854) (end 125.73 100.838) (width 0.25) (layer F.Cu) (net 2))
 (segment (start 125.73 100.838) (end 126.682 99.886) (width 0.25) (layer F.Cu) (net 2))
 (segment (start 126.682 99.886) (end 128.778 99.886) (width 0.25) (layer F.Cu) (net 2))
 (segment (start 147.066 101.534) (end 147.254 101.534) (width 0.25) (layer F.Cu) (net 2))
 (segment (start 150.368 107.188) (end 146.684 107.188) (width 0.25) (layer F.Cu) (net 2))
 (segment (start 146.684 107.188) (end 146.558 107.314) (width 0.25) (layer F.Cu) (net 2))
 (segment (start 135.66902 99.314) (end 137.602 99.314) (width 0.25) (layer F.Cu) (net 3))
 (segment (start 137.602 99.314) (end 137.668 99.38) (width 0.25) (layer F.Cu) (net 3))
 (segment (start 147.066 99.634) (end 148.148 99.634) (width 0.25) (layer F.Cu) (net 4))
 (segment (start 148.148 99.634) (end 150.368 101.854) (width 0.25) (layer F.Cu) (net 4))
 (segment (start 150.368 101.854) (end 150.368 102.108) (width 0.25) (layer F.Cu) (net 4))
 (segment (start 145.01622 100.584) (end 145.01622 99.83978) (width 0.25) (layer F.Cu) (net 4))
 (segment (start 145.222 99.634) (end 147.066 99.634) (width 0.25) (layer F.Cu) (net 4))
 (segment (start 145.01622 99.83978) (end 145.222 99.634) (width 0.25) (layer F.Cu) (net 4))
 (segment (start 150.368 99.568) (end 136.525 99.568) (width 0.25) (layer B.Cu) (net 5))
 (segment (start 131.699 104.394) (end 125.73 104.394) (width 0.25) (layer B.Cu) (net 5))
 (segment (start 136.525 99.568) (end 131.699 104.394) (width 0.25) (layer B.Cu) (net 5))
 (segment (start 125.73 104.394) (end 127.442 104.394) (width 0.25) (layer F.Cu) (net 5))
 (segment (start 127.442 104.394) (end 128.016 104.968) (width 0.25) (layer F.Cu) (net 5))
 (segment (start 141.412 101.473) (end 141.412 100.015) (width 0.25) (layer F.Cu) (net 6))
 (segment (start 141.793 99.634) (end 143.01724 99.634) (width 0.25) (layer F.Cu) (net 6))
 (segment (start 141.412 100.015) (end 141.793 99.634) (width 0.25) (layer F.Cu) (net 6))
 (segment (start 143.002 103.825) (end 143.002 103.632) (width 0.25) (layer F.Cu) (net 7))
 (segment (start 143.002 103.632) (end 144.018 102.616) (width 0.25) (layer F.Cu) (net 7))
 (segment (start 144.018 102.616) (end 144.018 98.933) (width 0.25) (layer F.Cu) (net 7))
 (segment (start 144.018 98.933) (end 143.637 98.552) (width 0.25) (layer F.Cu) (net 7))
 (segment (start 143.637 98.552) (end 141.478 98.552) (width 0.25) (layer F.Cu) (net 7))
 (segment (start 141.478 98.552) (end 140.589 99.441) (width 0.25) (layer F.Cu) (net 7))
 (segment (start 140.589 99.441) (end 139.319 99.441) (width 0.25) (layer F.Cu) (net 7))
 (segment (start 139.319 99.441) (end 138.43 100.33) (width 0.25) (layer F.Cu) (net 7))
 (segment (start 138.43 100.33) (end 136.779 100.33) (width 0.25) (layer F.Cu) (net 7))
 (segment (start 136.779 100.33) (end 136.525 100.584) (width 0.25) (layer F.Cu) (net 7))
 (segment (start 136.525 100.584) (end 136.525 104.902) (width 0.25) (layer F.Cu) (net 7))
 (segment (start 136.525 104.902) (end 136.017 105.41) (width 0.25) (layer F.Cu) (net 7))
 (segment (start 136.017 105.41) (end 135.222 105.41) (width 0.25) (layer F.Cu) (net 7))
 (segment (start 135.222 105.41) (end 135.095 105.537) (width 0.25) (layer F.Cu) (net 7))
 (segment (start 132.588 105.217) (end 132.903 105.217) (width 0.25) (layer F.Cu) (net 7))
 (segment (start 132.903 105.217) (end 133.223 105.537) (width 0.25) (layer F.Cu) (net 7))
 (segment (start 133.223 105.537) (end 135.095 105.537) (width 0.25) (layer F.Cu) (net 7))
 (segment (start 143.002 105.725) (end 143.002 105.537) (width 0.25) (layer F.Cu) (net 8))
 (segment (start 143.002 105.537) (end 143.764 104.775) (width 0.25) (layer F.Cu) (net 8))
 (segment (start 143.764 104.775) (end 144.847 104.775) (width 0.25) (layer F.Cu) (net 8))
 (segment (start 144.847 104.775) (end 145.558 104.064) (width 0.25) (layer F.Cu) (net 8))
 (segment (start 135.095 104.267) (end 135.095 103.538) (width 0.25) (layer F.Cu) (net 9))
 (segment (start 135.57 103.063) (end 135.57 101.346) (width 0.25) (layer F.Cu) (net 9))
 (segment (start 135.095 103.538) (end 135.57 103.063) (width 0.25) (layer F.Cu) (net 9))
 (segment (start 135.095 104.267) (end 131.318 104.267) (width 0.25) (layer F.Cu) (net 9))
 (segment (start 130.241 105.344) (end 130.241 107.569) (width 0.25) (layer F.Cu) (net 9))
 (segment (start 131.318 104.267) (end 130.241 105.344) (width 0.25) (layer F.Cu) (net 9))
 (segment (start 128.016 106.868) (end 128.016 107.315) (width 0.25) (layer F.Cu) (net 9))
 (segment (start 128.27 107.569) (end 130.241 107.569) (width 0.25) (layer F.Cu) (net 9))
 (segment (start 128.016 107.315) (end 128.27 107.569) (width 0.25) (layer F.Cu) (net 9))
 (segment (start 137.668 101.28) (end 139.319 101.28) (width 0.25) (layer F.Cu) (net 10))
 (segment (start 139.319 101.28) (end 139.512 101.473) (width 0.25) (layer F.Cu) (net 10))
 (segment (start 135.095 106.807) (end 136.144 106.807) (width 0.25) (layer F.Cu) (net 10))
 (segment (start 137.668 105.283) (end 137.668 101.28) (width 0.25) (layer F.Cu) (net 10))
 (segment (start 136.144 106.807) (end 137.668 105.283) (width 0.25) (layer F.Cu) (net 10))
 (segment (start 132.141 107.569) (end 132.842 107.569) (width 0.25) (layer F.Cu) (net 10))
 (segment (start 133.604 106.807) (end 135.095 106.807) (width 0.25) (layer F.Cu) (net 10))
 (segment (start 132.842 107.569) (end 133.604 106.807) (width 0.25) (layer F.Cu) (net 10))
 (segment (start 132.141 107.569) (end 132.334 107.569) (width 0.25) (layer F.Cu) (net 10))
 (segment (start 137.734 101.28) (end 137.668 101.28) (width 0.25) (layer F.Cu) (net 10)))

